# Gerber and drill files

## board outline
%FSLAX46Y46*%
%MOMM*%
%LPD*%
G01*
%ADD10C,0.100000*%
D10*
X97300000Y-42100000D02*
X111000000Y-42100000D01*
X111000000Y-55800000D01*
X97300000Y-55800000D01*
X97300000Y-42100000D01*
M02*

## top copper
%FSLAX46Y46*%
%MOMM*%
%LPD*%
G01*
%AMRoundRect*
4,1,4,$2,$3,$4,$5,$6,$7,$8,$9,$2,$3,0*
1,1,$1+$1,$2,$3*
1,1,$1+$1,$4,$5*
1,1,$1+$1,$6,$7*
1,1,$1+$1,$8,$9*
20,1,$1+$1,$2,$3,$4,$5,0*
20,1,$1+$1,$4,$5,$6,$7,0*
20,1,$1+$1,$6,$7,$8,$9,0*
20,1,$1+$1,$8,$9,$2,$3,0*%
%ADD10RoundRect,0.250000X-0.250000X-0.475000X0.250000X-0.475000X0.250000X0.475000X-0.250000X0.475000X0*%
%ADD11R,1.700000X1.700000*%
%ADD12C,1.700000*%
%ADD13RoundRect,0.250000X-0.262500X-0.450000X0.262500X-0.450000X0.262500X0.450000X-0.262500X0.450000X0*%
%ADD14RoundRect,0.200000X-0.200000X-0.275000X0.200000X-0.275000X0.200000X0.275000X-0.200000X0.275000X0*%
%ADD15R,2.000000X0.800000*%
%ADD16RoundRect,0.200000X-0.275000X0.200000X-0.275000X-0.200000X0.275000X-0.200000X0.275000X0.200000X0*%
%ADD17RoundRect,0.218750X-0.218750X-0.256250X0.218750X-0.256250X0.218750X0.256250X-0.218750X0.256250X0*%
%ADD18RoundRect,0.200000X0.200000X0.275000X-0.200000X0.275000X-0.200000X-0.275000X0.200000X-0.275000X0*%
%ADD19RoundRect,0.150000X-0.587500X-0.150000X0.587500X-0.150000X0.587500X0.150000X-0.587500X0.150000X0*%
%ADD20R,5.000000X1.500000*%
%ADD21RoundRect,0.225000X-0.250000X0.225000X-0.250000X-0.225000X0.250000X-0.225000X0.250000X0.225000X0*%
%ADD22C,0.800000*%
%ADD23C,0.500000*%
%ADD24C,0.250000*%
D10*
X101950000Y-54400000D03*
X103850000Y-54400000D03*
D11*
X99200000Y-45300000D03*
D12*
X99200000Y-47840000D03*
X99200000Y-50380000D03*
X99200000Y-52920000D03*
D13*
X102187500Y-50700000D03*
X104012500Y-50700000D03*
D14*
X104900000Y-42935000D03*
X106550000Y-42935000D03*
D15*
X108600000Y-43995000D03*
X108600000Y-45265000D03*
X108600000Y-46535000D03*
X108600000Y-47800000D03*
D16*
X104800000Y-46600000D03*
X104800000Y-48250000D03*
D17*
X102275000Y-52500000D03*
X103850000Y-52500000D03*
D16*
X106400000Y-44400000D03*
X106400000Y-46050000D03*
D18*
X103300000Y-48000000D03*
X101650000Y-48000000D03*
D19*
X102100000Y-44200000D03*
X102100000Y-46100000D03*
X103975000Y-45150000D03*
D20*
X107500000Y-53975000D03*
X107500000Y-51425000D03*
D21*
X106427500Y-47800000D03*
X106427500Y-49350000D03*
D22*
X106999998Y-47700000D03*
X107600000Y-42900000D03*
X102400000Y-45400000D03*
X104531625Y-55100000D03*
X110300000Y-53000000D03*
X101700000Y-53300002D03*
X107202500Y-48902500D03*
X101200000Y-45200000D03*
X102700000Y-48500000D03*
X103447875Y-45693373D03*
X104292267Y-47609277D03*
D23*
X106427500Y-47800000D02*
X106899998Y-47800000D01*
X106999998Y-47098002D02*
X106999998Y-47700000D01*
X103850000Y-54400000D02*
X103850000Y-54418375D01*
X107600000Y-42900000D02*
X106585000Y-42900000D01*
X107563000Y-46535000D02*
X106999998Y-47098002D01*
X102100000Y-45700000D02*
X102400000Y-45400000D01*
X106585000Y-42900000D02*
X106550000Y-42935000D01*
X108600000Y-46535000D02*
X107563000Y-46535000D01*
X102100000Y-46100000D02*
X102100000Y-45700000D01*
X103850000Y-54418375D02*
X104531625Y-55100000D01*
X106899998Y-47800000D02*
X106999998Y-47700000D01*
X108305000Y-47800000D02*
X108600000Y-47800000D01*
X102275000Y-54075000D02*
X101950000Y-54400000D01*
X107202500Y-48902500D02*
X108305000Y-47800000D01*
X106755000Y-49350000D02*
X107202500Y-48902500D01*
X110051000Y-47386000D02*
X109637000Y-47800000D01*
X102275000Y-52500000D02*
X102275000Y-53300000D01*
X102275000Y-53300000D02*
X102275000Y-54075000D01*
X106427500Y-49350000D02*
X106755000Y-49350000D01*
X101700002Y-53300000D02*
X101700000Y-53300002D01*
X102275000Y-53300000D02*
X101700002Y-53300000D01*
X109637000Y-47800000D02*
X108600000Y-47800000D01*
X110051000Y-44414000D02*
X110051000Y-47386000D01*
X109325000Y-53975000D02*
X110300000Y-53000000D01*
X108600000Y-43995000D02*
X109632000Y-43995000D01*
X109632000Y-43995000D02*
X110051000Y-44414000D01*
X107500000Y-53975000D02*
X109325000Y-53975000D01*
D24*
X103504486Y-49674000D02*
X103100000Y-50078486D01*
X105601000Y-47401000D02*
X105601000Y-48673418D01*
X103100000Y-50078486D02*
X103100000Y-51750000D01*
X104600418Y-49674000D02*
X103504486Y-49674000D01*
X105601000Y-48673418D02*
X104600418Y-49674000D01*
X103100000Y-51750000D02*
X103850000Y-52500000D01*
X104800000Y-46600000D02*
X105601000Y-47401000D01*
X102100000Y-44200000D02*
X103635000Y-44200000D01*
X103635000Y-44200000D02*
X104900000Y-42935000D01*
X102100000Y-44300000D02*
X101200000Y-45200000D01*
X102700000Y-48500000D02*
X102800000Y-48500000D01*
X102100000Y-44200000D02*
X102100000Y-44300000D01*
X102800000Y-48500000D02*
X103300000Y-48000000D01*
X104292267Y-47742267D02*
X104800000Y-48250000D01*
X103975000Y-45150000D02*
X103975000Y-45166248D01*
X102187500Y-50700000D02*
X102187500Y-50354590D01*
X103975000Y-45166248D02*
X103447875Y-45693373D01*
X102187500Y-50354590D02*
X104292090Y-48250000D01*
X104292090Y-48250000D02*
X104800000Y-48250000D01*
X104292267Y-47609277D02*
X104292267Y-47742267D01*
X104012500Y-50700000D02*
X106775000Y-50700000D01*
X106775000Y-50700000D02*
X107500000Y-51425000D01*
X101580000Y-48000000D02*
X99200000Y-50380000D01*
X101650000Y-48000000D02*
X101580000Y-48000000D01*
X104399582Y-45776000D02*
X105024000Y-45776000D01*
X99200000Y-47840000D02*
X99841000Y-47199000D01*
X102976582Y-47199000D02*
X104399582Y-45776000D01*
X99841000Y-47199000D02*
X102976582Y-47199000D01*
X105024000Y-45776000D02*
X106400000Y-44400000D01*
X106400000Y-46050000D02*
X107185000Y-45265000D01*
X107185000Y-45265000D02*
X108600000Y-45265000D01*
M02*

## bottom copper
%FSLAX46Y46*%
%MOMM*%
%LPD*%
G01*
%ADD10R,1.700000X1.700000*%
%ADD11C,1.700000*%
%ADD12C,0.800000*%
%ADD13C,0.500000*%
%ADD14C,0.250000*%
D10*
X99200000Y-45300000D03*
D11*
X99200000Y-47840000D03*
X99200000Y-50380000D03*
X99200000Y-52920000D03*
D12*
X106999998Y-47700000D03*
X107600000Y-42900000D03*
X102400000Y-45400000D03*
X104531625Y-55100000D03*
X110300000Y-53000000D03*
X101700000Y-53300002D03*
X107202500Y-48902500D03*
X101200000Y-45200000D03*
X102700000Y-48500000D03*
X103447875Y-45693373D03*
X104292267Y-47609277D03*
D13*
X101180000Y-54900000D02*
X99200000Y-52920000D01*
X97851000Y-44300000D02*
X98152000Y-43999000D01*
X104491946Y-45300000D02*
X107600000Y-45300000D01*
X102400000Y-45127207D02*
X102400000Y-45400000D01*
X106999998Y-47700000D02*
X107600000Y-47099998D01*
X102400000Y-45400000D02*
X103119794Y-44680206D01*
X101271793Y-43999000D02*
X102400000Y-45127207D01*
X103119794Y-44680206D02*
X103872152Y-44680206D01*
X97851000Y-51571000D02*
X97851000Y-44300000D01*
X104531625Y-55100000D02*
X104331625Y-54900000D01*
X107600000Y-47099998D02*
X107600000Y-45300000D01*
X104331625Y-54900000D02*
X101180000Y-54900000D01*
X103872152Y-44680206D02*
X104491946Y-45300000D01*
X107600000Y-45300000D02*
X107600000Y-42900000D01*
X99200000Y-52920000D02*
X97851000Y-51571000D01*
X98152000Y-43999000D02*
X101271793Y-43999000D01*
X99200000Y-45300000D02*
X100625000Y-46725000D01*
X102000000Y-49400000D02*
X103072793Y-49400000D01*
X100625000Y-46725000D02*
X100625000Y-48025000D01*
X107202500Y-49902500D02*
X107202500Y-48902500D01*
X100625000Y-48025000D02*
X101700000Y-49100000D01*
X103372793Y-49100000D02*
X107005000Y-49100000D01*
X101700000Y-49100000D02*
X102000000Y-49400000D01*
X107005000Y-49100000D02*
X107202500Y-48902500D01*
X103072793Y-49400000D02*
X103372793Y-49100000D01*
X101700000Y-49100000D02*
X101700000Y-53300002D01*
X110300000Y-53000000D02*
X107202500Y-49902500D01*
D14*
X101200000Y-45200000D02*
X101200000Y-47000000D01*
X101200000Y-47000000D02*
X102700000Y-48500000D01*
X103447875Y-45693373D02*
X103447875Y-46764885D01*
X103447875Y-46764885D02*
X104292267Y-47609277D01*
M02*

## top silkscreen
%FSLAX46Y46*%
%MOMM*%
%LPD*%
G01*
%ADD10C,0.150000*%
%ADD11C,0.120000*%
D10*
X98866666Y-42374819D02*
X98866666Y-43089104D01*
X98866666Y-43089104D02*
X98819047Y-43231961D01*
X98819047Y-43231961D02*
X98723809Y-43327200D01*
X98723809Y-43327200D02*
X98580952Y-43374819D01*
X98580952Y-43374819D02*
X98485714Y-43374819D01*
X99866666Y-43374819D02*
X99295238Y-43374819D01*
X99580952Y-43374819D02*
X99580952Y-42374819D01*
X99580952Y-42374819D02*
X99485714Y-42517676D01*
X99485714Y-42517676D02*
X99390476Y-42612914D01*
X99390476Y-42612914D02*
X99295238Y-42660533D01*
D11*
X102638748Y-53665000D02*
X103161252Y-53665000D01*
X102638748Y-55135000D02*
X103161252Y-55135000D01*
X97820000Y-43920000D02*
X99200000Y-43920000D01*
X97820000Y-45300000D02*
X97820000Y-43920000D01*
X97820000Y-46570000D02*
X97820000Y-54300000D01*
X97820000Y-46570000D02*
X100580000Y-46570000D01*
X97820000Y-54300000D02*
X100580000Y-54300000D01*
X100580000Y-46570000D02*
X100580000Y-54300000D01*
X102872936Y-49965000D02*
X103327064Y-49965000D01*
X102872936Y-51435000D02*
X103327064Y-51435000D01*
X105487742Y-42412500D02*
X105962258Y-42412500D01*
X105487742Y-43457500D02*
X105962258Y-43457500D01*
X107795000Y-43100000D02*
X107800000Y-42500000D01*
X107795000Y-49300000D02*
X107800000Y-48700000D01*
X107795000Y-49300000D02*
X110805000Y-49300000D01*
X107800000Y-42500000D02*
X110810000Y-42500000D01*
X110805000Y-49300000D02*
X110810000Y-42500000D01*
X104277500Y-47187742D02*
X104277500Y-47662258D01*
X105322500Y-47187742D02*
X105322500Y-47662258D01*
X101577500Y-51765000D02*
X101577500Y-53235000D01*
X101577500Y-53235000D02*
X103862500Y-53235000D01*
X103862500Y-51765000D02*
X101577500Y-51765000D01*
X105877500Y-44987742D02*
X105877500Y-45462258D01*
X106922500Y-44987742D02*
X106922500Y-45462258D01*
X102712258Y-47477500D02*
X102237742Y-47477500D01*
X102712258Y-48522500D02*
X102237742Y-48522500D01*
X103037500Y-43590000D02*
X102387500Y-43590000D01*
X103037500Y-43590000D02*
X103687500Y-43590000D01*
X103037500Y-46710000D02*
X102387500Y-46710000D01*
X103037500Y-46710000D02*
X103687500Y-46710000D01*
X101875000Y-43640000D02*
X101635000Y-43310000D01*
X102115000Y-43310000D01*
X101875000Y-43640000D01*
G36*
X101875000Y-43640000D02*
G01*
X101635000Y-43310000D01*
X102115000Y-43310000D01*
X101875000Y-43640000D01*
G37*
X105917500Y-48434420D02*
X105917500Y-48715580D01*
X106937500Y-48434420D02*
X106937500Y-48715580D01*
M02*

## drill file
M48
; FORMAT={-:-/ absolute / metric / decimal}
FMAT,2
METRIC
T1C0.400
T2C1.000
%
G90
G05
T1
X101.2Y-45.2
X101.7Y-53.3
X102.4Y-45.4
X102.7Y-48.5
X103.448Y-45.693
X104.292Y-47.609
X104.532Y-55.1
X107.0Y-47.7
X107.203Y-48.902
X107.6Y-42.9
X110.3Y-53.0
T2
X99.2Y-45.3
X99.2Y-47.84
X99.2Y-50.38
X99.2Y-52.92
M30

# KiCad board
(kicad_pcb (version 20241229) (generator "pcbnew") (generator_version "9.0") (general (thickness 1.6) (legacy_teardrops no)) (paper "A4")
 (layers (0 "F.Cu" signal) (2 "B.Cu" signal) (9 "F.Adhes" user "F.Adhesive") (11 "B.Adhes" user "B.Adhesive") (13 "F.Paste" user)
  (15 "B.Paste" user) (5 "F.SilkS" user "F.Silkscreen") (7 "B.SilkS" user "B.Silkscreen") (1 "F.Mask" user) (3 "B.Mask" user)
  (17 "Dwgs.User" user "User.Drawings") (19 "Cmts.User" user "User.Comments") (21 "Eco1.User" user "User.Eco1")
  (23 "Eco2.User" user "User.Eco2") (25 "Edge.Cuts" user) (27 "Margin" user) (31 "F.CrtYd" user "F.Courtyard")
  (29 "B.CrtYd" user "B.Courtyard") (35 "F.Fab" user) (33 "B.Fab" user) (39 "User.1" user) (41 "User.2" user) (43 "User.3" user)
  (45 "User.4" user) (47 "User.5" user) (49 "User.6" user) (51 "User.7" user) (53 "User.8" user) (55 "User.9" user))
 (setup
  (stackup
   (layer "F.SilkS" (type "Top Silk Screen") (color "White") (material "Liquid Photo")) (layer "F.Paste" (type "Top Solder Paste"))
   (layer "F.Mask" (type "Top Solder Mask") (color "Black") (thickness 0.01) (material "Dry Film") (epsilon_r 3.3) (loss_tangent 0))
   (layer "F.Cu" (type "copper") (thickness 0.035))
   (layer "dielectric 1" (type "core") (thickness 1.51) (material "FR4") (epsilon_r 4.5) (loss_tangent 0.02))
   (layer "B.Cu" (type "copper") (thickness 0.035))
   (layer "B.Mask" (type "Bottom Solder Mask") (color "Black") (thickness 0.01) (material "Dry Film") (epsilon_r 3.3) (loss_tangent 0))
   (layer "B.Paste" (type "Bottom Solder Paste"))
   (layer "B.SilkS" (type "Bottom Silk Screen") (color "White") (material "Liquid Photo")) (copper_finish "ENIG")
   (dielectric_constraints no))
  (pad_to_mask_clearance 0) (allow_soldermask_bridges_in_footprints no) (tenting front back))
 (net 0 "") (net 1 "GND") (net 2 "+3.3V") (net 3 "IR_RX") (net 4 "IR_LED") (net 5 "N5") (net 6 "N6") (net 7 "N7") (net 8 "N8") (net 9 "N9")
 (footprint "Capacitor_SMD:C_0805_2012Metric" (layer "F.Cu") (at 102.9 54.4)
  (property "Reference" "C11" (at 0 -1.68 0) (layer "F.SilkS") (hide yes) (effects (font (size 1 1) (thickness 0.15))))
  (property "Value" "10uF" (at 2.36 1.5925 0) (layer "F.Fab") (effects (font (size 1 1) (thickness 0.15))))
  (fp_line (start -0.261252 -0.735) (end 0.261252 -0.735) (stroke (width 0.12) (type solid)) (layer "F.SilkS"))
  (fp_line (start -0.261252 0.735) (end 0.261252 0.735) (stroke (width 0.12) (type solid)) (layer "F.SilkS"))
  (pad "1" smd roundrect (at -0.95 0) (size 1 1.45) (layers "F.Cu" "F.Mask" "F.Paste") (roundrect_rratio 0.25) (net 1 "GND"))
  (pad "2" smd roundrect (at 0.95 0) (size 1 1.45) (layers "F.Cu" "F.Mask" "F.Paste") (roundrect_rratio 0.25) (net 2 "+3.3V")))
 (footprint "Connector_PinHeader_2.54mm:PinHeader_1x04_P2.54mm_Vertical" (layer "F.Cu") (at 99.2 45.3)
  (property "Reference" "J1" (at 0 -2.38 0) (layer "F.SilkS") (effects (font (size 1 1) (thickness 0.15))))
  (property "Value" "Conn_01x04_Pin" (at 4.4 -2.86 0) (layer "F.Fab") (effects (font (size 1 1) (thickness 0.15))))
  (fp_line (start -1.38 -1.38) (end 0 -1.38) (stroke (width 0.12) (type solid)) (layer "F.SilkS"))
  (fp_line (start -1.38 0) (end -1.38 -1.38) (stroke (width 0.12) (type solid)) (layer "F.SilkS"))
  (fp_line (start -1.38 1.27) (end -1.38 9) (stroke (width 0.12) (type solid)) (layer "F.SilkS"))
  (fp_line (start -1.38 1.27) (end 1.38 1.27) (stroke (width 0.12) (type solid)) (layer "F.SilkS"))
  (fp_line (start -1.38 9) (end 1.38 9) (stroke (width 0.12) (type solid)) (layer "F.SilkS"))
  (fp_line (start 1.38 1.27) (end 1.38 9) (stroke (width 0.12) (type solid)) (layer "F.SilkS"))
  (pad "1" thru_hole rect (at 0 0) (size 1.7 1.7) (drill 1) (layers "*.Cu" "*.Mask") (remove_unused_layers no) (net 1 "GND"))
  (pad "2" thru_hole circle (at 0 2.54) (size 1.7 1.7) (drill 1) (layers "*.Cu" "*.Mask") (remove_unused_layers no) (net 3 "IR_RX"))
  (pad "3" thru_hole circle (at 0 5.08) (size 1.7 1.7) (drill 1) (layers "*.Cu" "*.Mask") (remove_unused_layers no) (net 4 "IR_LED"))
  (pad "4" thru_hole circle (at 0 7.62) (size 1.7 1.7) (drill 1) (layers "*.Cu" "*.Mask") (remove_unused_layers no) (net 2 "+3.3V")))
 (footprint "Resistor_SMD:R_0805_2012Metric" (layer "F.Cu") (at 103.1 50.7)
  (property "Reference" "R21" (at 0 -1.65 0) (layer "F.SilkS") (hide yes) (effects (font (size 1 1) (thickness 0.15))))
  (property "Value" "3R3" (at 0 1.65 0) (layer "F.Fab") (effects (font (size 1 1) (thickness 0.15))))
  (fp_line (start -0.227064 -0.735) (end 0.227064 -0.735) (stroke (width 0.12) (type solid)) (layer "F.SilkS"))
  (fp_line (start -0.227064 0.735) (end 0.227064 0.735) (stroke (width 0.12) (type solid)) (layer "F.SilkS"))
  (pad "1" smd roundrect (at -0.9125 0) (size 1.025 1.4) (layers "F.Cu" "F.Mask" "F.Paste") (roundrect_rratio 0.243902) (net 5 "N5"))
  (pad "2" smd roundrect (at 0.9125 0) (size 1.025 1.4) (layers "F.Cu" "F.Mask" "F.Paste") (roundrect_rratio 0.243902) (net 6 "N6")))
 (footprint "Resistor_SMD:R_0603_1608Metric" (layer "F.Cu") (at 105.725 42.935)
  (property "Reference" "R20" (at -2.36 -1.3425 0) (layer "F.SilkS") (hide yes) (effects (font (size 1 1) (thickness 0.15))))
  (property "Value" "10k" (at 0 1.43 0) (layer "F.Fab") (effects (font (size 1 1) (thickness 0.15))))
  (fp_line (start -0.237258 -0.5225) (end 0.237258 -0.5225) (stroke (width 0.12) (type solid)) (layer "F.SilkS"))
  (fp_line (start -0.237258 0.5225) (end 0.237258 0.5225) (stroke (width 0.12) (type solid)) (layer "F.SilkS"))
  (pad "1" smd roundrect (at -0.825 0) (size 0.8 0.95) (layers "F.Cu" "F.Mask" "F.Paste") (roundrect_rratio 0.25) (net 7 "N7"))
  (pad "2" smd roundrect (at 0.825 0) (size 0.8 0.95) (layers "F.Cu" "F.Mask" "F.Paste") (roundrect_rratio 0.25) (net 2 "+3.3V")))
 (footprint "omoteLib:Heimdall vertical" (layer "F.Cu") (at 109.3 45.9 -90)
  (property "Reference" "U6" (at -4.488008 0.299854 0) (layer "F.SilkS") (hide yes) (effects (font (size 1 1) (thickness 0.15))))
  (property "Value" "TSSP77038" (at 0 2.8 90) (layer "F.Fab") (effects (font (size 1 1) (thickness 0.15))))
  (fp_line (start -2.8 1.505) (end -3.4 1.5) (stroke (width 0.12) (type solid)) (layer "F.SilkS"))
  (fp_line (start 3.4 1.505) (end 2.8 1.5) (stroke (width 0.12) (type solid)) (layer "F.SilkS"))
  (fp_line (start 3.4 1.505) (end 3.4 -1.505) (stroke (width 0.12) (type solid)) (layer "F.SilkS"))
  (fp_line (start -3.4 1.5) (end -3.4 -1.51) (stroke (width 0.12) (type solid)) (layer "F.SilkS"))
  (fp_line (start 3.4 -1.505) (end -3.4 -1.51) (stroke (width 0.12) (type solid)) (layer "F.SilkS"))
  (pad "1" smd rect (at -1.905 0.7) (size 2 0.8) (layers "F.Cu" "F.Mask" "F.Paste") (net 1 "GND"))
  (pad "2" smd rect (at -0.635 0.7) (size 2 0.8) (layers "F.Cu" "F.Mask" "F.Paste") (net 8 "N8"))
  (pad "3" smd rect (at 0.635 0.7) (size 2 0.8) (layers "F.Cu" "F.Mask" "F.Paste") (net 2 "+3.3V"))
  (pad "4" smd rect (at 1.9 0.7) (size 2 0.8) (layers "F.Cu" "F.Mask" "F.Paste") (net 1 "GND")))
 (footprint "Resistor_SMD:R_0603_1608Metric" (layer "F.Cu") (at 104.8 47.425 -90)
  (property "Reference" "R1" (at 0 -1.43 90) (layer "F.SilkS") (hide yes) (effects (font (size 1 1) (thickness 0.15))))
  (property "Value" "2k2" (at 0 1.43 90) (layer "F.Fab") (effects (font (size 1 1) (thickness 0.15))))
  (fp_line (start -0.237258 0.5225) (end 0.237258 0.5225) (stroke (width 0.12) (type solid)) (layer "F.SilkS"))
  (fp_line (start -0.237258 -0.5225) (end 0.237258 -0.5225) (stroke (width 0.12) (type solid)) (layer "F.SilkS"))
  (pad "1" smd roundrect (at -0.825 0 270) (size 0.8 0.95) (layers "F.Cu" "F.Mask" "F.Paste") (roundrect_rratio 0.25) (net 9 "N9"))
  (pad "2" smd roundrect (at 0.825 0 270) (size 0.8 0.95) (layers "F.Cu" "F.Mask" "F.Paste") (roundrect_rratio 0.25) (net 5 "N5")))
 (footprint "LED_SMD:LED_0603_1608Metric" (layer "F.Cu") (at 103.0625 52.5)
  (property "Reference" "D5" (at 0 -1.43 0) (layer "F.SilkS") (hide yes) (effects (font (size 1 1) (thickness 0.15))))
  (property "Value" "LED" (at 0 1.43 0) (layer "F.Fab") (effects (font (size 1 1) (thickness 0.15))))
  (fp_line (start -1.485 -0.735) (end -1.485 0.735) (stroke (width 0.12) (type solid)) (layer "F.SilkS"))
  (fp_line (start -1.485 0.735) (end 0.8 0.735) (stroke (width 0.12) (type solid)) (layer "F.SilkS"))
  (fp_line (start 0.8 -0.735) (end -1.485 -0.735) (stroke (width 0.12) (type solid)) (layer "F.SilkS"))
  (pad "1" smd roundrect (at -0.7875 0) (size 0.875 0.95) (layers "F.Cu" "F.Mask" "F.Paste") (roundrect_rratio 0.25) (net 1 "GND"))
  (pad "2" smd roundrect (at 0.7875 0) (size 0.875 0.95) (layers "F.Cu" "F.Mask" "F.Paste") (roundrect_rratio 0.25) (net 9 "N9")))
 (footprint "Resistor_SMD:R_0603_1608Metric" (layer "F.Cu") (at 106.4 45.225 -90)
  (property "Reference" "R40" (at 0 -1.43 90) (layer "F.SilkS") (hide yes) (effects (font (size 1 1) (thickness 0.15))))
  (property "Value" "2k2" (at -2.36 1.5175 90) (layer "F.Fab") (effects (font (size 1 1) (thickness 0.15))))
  (fp_line (start -0.237258 0.5225) (end 0.237258 0.5225) (stroke (width 0.12) (type solid)) (layer "F.SilkS"))
  (fp_line (start -0.237258 -0.5225) (end 0.237258 -0.5225) (stroke (width 0.12) (type solid)) (layer "F.SilkS"))
  (pad "1" smd roundrect (at -0.825 0 270) (size 0.8 0.95) (layers "F.Cu" "F.Mask" "F.Paste") (roundrect_rratio 0.25) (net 3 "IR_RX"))
  (pad "2" smd roundrect (at 0.825 0 270) (size 0.8 0.95) (layers "F.Cu" "F.Mask" "F.Paste") (roundrect_rratio 0.25) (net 8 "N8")))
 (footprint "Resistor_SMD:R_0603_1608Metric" (layer "F.Cu") (at 102.475 48 180)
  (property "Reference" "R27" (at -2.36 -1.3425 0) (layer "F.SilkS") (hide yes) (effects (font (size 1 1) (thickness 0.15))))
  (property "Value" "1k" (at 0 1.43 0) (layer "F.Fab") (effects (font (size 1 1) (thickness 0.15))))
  (fp_line (start -0.237258 0.5225) (end 0.237258 0.5225) (stroke (width 0.12) (type solid)) (layer "F.SilkS"))
  (fp_line (start -0.237258 -0.5225) (end 0.237258 -0.5225) (stroke (width 0.12) (type solid)) (layer "F.SilkS"))
  (pad "1" smd roundrect (at -0.825 0 180) (size 0.8 0.95) (layers "F.Cu" "F.Mask" "F.Paste") (roundrect_rratio 0.25) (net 7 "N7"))
  (pad "2" smd roundrect (at 0.825 0 180) (size 0.8 0.95) (layers "F.Cu" "F.Mask" "F.Paste") (roundrect_rratio 0.25) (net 4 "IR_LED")))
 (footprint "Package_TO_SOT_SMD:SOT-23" (layer "F.Cu") (at 103.0375 45.15)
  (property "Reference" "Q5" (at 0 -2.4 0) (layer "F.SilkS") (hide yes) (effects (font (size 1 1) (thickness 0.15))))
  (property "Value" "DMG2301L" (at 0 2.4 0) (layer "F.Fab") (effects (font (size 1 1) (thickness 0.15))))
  (fp_line (start 0 -1.56) (end -0.65 -1.56) (stroke (width 0.12) (type solid)) (layer "F.SilkS"))
  (fp_line (start 0 -1.56) (end 0.65 -1.56) (stroke (width 0.12) (type solid)) (layer "F.SilkS"))
  (fp_line (start 0 1.56) (end -0.65 1.56) (stroke (width 0.12) (type solid)) (layer "F.SilkS"))
  (fp_line (start 0 1.56) (end 0.65 1.56) (stroke (width 0.12) (type solid)) (layer "F.SilkS"))
  (fp_poly (pts (xy -1.1625 -1.51) (xy -1.4025 -1.84) (xy -0.9225 -1.84)) (stroke (width 0.12) (type solid)) (fill yes) (layer "F.SilkS"))
  (pad "1" smd roundrect (at -0.9375 -0.95) (size 1.475 0.6) (layers "F.Cu" "F.Mask" "F.Paste") (roundrect_rratio 0.25) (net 7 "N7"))
  (pad "2" smd roundrect (at -0.9375 0.95) (size 1.475 0.6) (layers "F.Cu" "F.Mask" "F.Paste") (roundrect_rratio 0.25) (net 2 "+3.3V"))
  (pad "3" smd roundrect (at 0.9375 0) (size 1.475 0.6) (layers "F.Cu" "F.Mask" "F.Paste") (roundrect_rratio 0.25) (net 5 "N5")))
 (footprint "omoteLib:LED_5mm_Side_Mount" (layer "F.Cu") (at 111 52.7 -90)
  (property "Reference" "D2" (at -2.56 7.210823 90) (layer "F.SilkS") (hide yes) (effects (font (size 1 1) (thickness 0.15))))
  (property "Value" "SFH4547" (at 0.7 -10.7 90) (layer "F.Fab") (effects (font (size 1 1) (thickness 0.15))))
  (pad "1" smd rect (at 1.275 3.5 270) (size 1.5 5) (layers "F.Cu" "F.Mask" "F.Paste") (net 1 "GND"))
  (pad "2" smd rect (at -1.275 3.5 270) (size 1.5 5) (layers "F.Cu" "F.Mask" "F.Paste") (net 6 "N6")))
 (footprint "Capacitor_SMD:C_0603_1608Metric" (layer "F.Cu") (at 106.4275 48.575 -90)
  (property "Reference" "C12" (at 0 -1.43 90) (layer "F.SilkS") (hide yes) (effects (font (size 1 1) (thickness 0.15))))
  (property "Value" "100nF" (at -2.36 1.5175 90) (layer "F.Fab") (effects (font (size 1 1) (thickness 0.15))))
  (fp_line (start -0.14058 0.51) (end 0.14058 0.51) (stroke (width 0.12) (type solid)) (layer "F.SilkS"))
  (fp_line (start -0.14058 -0.51) (end 0.14058 -0.51) (stroke (width 0.12) (type solid)) (layer "F.SilkS"))
  (pad "1" smd roundrect (at -0.775 0 270) (size 0.9 0.95) (layers "F.Cu" "F.Mask" "F.Paste") (roundrect_rratio 0.25) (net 2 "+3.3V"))
  (pad "2" smd roundrect (at 0.775 0 270) (size 0.9 0.95) (layers "F.Cu" "F.Mask" "F.Paste") (roundrect_rratio 0.25) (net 1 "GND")))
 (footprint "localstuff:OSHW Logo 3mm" (layer "B.Cu") (at 107.5 52.8 180)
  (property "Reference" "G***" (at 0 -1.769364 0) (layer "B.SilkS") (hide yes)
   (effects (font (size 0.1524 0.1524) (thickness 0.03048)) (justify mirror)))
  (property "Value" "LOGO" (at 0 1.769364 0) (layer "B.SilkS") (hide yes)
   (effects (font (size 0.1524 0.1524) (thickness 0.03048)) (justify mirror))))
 (gr_rect (start 97.3 42.1) (end 111 55.8) (stroke (width 0.1) (type default)) (fill no) (layer "Edge.Cuts"))
 (segment (start 106.4275 47.8) (end 106.899998 47.8) (width 0.5) (layer "F.Cu") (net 2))
 (segment (start 106.999998 47.098002) (end 106.999998 47.7) (width 0.5) (layer "F.Cu") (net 2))
 (segment (start 103.85 54.4) (end 103.85 54.418375) (width 0.5) (layer "F.Cu") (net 2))
 (segment (start 107.6 42.9) (end 106.585 42.9) (width 0.5) (layer "F.Cu") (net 2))
 (segment (start 107.563 46.535) (end 106.999998 47.098002) (width 0.5) (layer "F.Cu") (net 2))
 (segment (start 102.1 45.7) (end 102.4 45.4) (width 0.5) (layer "F.Cu") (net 2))
 (segment (start 106.585 42.9) (end 106.55 42.935) (width 0.5) (layer "F.Cu") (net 2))
 (segment (start 108.6 46.535) (end 107.563 46.535) (width 0.5) (layer "F.Cu") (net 2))
 (segment (start 102.1 46.1) (end 102.1 45.7) (width 0.5) (layer "F.Cu") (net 2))
 (segment (start 103.85 54.418375) (end 104.531625 55.1) (width 0.5) (layer "F.Cu") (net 2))
 (segment (start 106.899998 47.8) (end 106.999998 47.7) (width 0.5) (layer "F.Cu") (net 2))
 (via (at 106.999998 47.7) (size 0.8) (drill 0.4) (layers "F.Cu" "B.Cu") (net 2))
 (via (at 107.6 42.9) (size 0.8) (drill 0.4) (layers "F.Cu" "B.Cu") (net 2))
 (via (at 102.4 45.4) (size 0.8) (drill 0.4) (layers "F.Cu" "B.Cu") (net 2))
 (via (at 104.531625 55.1) (size 0.8) (drill 0.4) (layers "F.Cu" "B.Cu") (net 2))
 (segment (start 101.18 54.9) (end 99.2 52.92) (width 0.5) (layer "B.Cu") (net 2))
 (segment (start 97.851 44.3) (end 98.152 43.999) (width 0.5) (layer "B.Cu") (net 2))
 (segment (start 104.491946 45.3) (end 107.6 45.3) (width 0.5) (layer "B.Cu") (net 2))
 (segment (start 102.4 45.127207) (end 102.4 45.4) (width 0.5) (layer "B.Cu") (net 2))
 (segment (start 106.999998 47.7) (end 107.6 47.099998) (width 0.5) (layer "B.Cu") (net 2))
 (segment (start 102.4 45.4) (end 103.119794 44.680206) (width 0.5) (layer "B.Cu") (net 2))
 (segment (start 101.271793 43.999) (end 102.4 45.127207) (width 0.5) (layer "B.Cu") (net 2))
 (segment (start 103.119794 44.680206) (end 103.872152 44.680206) (width 0.5) (layer "B.Cu") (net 2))
 (segment (start 97.851 51.571) (end 97.851 44.3) (width 0.5) (layer "B.Cu") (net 2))
 (segment (start 104.531625 55.1) (end 104.331625 54.9) (width 0.5) (layer "B.Cu") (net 2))
 (segment (start 107.6 47.099998) (end 107.6 45.3) (width 0.5) (layer "B.Cu") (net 2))
 (segment (start 104.331625 54.9) (end 101.18 54.9) (width 0.5) (layer "B.Cu") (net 2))
 (segment (start 103.872152 44.680206) (end 104.491946 45.3) (width 0.5) (layer "B.Cu") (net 2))
 (segment (start 107.6 45.3) (end 107.6 42.9) (width 0.5) (layer "B.Cu") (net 2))
 (segment (start 99.2 52.92) (end 97.851 51.571) (width 0.5) (layer "B.Cu") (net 2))
 (segment (start 98.152 43.999) (end 101.271793 43.999) (width 0.5) (layer "B.Cu") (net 2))
 (segment (start 108.305 47.8) (end 108.6 47.8) (width 0.5) (layer "F.Cu") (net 1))
 (segment (start 102.275 54.075) (end 101.95 54.4) (width 0.5) (layer "F.Cu") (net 1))
 (segment (start 107.2025 48.9025) (end 108.305 47.8) (width 0.5) (layer "F.Cu") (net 1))
 (segment (start 106.755 49.35) (end 107.2025 48.9025) (width 0.5) (layer "F.Cu") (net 1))
 (segment (start 110.051 47.386) (end 109.637 47.8) (width 0.5) (layer "F.Cu") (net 1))
 (segment (start 102.275 52.5) (end 102.275 53.3) (width 0.5) (layer "F.Cu") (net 1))
 (segment (start 102.275 53.3) (end 102.275 54.075) (width 0.5) (layer "F.Cu") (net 1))
 (segment (start 106.4275 49.35) (end 106.755 49.35) (width 0.5) (layer "F.Cu") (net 1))
 (segment (start 101.700002 53.3) (end 101.7 53.300002) (width 0.5) (layer "F.Cu") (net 1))
 (segment (start 102.275 53.3) (end 101.700002 53.3) (width 0.5) (layer "F.Cu") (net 1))
 (segment (start 109.637 47.8) (end 108.6 47.8) (width 0.5) (layer "F.Cu") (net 1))
 (segment (start 110.051 44.414) (end 110.051 47.386) (width 0.5) (layer "F.Cu") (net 1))
 (segment (start 109.325 53.975) (end 110.3 53) (width 0.5) (layer "F.Cu") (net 1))
 (segment (start 108.6 43.995) (end 109.632 43.995) (width 0.5) (layer "F.Cu") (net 1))
 (segment (start 109.632 43.995) (end 110.051 44.414) (width 0.5) (layer "F.Cu") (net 1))
 (segment (start 107.5 53.975) (end 109.325 53.975) (width 0.5) (layer "F.Cu") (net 1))
 (via (at 110.3 53) (size 0.8) (drill 0.4) (layers "F.Cu" "B.Cu") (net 1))
 (via (at 101.7 53.300002) (size 0.8) (drill 0.4) (layers "F.Cu" "B.Cu") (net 1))
 (via (at 107.2025 48.9025) (size 0.8) (drill 0.4) (layers "F.Cu" "B.Cu") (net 1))
 (segment (start 99.2 45.3) (end 100.625 46.725) (width 0.5) (layer "B.Cu") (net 1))
 (segment (start 102 49.4) (end 103.072793 49.4) (width 0.5) (layer "B.Cu") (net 1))
 (segment (start 100.625 46.725) (end 100.625 48.025) (width 0.5) (layer "B.Cu") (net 1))
 (segment (start 107.2025 49.9025) (end 107.2025 48.9025) (width 0.5) (layer "B.Cu") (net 1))
 (segment (start 100.625 48.025) (end 101.7 49.1) (width 0.5) (layer "B.Cu") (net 1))
 (segment (start 103.372793 49.1) (end 107.005 49.1) (width 0.5) (layer "B.Cu") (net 1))
 (segment (start 101.7 49.1) (end 102 49.4) (width 0.5) (layer "B.Cu") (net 1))
 (segment (start 107.005 49.1) (end 107.2025 48.9025) (width 0.5) (layer "B.Cu") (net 1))
 (segment (start 103.072793 49.4) (end 103.372793 49.1) (width 0.5) (layer "B.Cu") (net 1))
 (segment (start 101.7 49.1) (end 101.7 53.300002) (width 0.5) (layer "B.Cu") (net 1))
 (segment (start 110.3 53) (end 107.2025 49.9025) (width 0.5) (layer "B.Cu") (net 1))
 (segment (start 103.504486 49.674) (end 103.1 50.078486) (width 0.25) (layer "F.Cu") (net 9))
 (segment (start 105.601 47.401) (end 105.601 48.673418) (width 0.25) (layer "F.Cu") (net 9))
 (segment (start 103.1 50.078486) (end 103.1 51.75) (width 0.25) (layer "F.Cu") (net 9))
 (segment (start 104.600418 49.674) (end 103.504486 49.674) (width 0.25) (layer "F.Cu") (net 9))
 (segment (start 105.601 48.673418) (end 104.600418 49.674) (width 0.25) (layer "F.Cu") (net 9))
 (segment (start 103.1 51.75) (end 103.85 52.5) (width 0.25) (layer "F.Cu") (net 9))
 (segment (start 104.8 46.6) (end 105.601 47.401) (width 0.25) (layer "F.Cu") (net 9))
 (segment (start 102.1 44.2) (end 103.635 44.2) (width 0.25) (layer "F.Cu") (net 7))
 (segment (start 103.635 44.2) (end 104.9 42.935) (width 0.25) (layer "F.Cu") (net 7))
 (segment (start 102.1 44.3) (end 101.2 45.2) (width 0.25) (layer "F.Cu") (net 7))
 (segment (start 102.7 48.5) (end 102.8 48.5) (width 0.25) (layer "F.Cu") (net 7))
 (segment (start 102.1 44.2) (end 102.1 44.3) (width 0.25) (layer "F.Cu") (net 7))
 (segment (start 102.8 48.5) (end 103.3 48) (width 0.25) (layer "F.Cu") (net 7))
 (via (at 101.2 45.2) (size 0.8) (drill 0.4) (layers "F.Cu" "B.Cu") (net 7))
 (via (at 102.7 48.5) (size 0.8) (drill 0.4) (layers "F.Cu" "B.Cu") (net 7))
 (segment (start 101.2 45.2) (end 101.2 47) (width 0.25) (layer "B.Cu") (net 7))
 (segment (start 101.2 47) (end 102.7 48.5) (width 0.25) (layer "B.Cu") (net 7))
 (segment (start 104.292267 47.742267) (end 104.8 48.25) (width 0.25) (layer "F.Cu") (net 5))
 (segment (start 103.975 45.15) (end 103.975 45.166248) (width 0.25) (layer "F.Cu") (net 5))
 (segment (start 102.1875 50.7) (end 102.1875 50.35459) (width 0.25) (layer "F.Cu") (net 5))
 (segment (start 103.975 45.166248) (end 103.447875 45.693373) (width 0.25) (layer "F.Cu") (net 5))
 (segment (start 102.1875 50.35459) (end 104.29209 48.25) (width 0.25) (layer "F.Cu") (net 5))
 (segment (start 104.29209 48.25) (end 104.8 48.25) (width 0.25) (layer "F.Cu") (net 5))
 (segment (start 104.292267 47.609277) (end 104.292267 47.742267) (width 0.25) (layer "F.Cu") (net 5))
 (via (at 103.447875 45.693373) (size 0.8) (drill 0.4) (layers "F.Cu" "B.Cu") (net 5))
 (via (at 104.292267 47.609277) (size 0.8) (drill 0.4) (layers "F.Cu" "B.Cu") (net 5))
 (segment (start 103.447875 45.693373) (end 103.447875 46.764885) (width 0.25) (layer "B.Cu") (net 5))
 (segment (start 103.447875 46.764885) (end 104.292267 47.609277) (width 0.25) (layer "B.Cu") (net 5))
 (segment (start 104.0125 50.7) (end 106.775 50.7) (width 0.25) (layer "F.Cu") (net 6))
 (segment (start 106.775 50.7) (end 107.5 51.425) (width 0.25) (layer "F.Cu") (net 6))
 (segment (start 101.58 48) (end 99.2 50.38) (width 0.25) (layer "F.Cu") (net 4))
 (segment (start 101.65 48) (end 101.58 48) (width 0.25) (layer "F.Cu") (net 4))
 (segment (start 104.399582 45.776) (end 105.024 45.776) (width 0.25) (layer "F.Cu") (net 3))
 (segment (start 99.2 47.84) (end 99.841 47.199) (width 0.25) (layer "F.Cu") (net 3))
 (segment (start 102.976582 47.199) (end 104.399582 45.776) (width 0.25) (layer "F.Cu") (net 3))
 (segment (start 99.841 47.199) (end 102.976582 47.199) (width 0.25) (layer "F.Cu") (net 3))
 (segment (start 105.024 45.776) (end 106.4 44.4) (width 0.25) (layer "F.Cu") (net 3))
 (segment (start 106.4 46.05) (end 107.185 45.265) (width 0.25) (layer "F.Cu") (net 8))
 (segment (start 107.185 45.265) (end 108.6 45.265) (width 0.25) (layer "F.Cu") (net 8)))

